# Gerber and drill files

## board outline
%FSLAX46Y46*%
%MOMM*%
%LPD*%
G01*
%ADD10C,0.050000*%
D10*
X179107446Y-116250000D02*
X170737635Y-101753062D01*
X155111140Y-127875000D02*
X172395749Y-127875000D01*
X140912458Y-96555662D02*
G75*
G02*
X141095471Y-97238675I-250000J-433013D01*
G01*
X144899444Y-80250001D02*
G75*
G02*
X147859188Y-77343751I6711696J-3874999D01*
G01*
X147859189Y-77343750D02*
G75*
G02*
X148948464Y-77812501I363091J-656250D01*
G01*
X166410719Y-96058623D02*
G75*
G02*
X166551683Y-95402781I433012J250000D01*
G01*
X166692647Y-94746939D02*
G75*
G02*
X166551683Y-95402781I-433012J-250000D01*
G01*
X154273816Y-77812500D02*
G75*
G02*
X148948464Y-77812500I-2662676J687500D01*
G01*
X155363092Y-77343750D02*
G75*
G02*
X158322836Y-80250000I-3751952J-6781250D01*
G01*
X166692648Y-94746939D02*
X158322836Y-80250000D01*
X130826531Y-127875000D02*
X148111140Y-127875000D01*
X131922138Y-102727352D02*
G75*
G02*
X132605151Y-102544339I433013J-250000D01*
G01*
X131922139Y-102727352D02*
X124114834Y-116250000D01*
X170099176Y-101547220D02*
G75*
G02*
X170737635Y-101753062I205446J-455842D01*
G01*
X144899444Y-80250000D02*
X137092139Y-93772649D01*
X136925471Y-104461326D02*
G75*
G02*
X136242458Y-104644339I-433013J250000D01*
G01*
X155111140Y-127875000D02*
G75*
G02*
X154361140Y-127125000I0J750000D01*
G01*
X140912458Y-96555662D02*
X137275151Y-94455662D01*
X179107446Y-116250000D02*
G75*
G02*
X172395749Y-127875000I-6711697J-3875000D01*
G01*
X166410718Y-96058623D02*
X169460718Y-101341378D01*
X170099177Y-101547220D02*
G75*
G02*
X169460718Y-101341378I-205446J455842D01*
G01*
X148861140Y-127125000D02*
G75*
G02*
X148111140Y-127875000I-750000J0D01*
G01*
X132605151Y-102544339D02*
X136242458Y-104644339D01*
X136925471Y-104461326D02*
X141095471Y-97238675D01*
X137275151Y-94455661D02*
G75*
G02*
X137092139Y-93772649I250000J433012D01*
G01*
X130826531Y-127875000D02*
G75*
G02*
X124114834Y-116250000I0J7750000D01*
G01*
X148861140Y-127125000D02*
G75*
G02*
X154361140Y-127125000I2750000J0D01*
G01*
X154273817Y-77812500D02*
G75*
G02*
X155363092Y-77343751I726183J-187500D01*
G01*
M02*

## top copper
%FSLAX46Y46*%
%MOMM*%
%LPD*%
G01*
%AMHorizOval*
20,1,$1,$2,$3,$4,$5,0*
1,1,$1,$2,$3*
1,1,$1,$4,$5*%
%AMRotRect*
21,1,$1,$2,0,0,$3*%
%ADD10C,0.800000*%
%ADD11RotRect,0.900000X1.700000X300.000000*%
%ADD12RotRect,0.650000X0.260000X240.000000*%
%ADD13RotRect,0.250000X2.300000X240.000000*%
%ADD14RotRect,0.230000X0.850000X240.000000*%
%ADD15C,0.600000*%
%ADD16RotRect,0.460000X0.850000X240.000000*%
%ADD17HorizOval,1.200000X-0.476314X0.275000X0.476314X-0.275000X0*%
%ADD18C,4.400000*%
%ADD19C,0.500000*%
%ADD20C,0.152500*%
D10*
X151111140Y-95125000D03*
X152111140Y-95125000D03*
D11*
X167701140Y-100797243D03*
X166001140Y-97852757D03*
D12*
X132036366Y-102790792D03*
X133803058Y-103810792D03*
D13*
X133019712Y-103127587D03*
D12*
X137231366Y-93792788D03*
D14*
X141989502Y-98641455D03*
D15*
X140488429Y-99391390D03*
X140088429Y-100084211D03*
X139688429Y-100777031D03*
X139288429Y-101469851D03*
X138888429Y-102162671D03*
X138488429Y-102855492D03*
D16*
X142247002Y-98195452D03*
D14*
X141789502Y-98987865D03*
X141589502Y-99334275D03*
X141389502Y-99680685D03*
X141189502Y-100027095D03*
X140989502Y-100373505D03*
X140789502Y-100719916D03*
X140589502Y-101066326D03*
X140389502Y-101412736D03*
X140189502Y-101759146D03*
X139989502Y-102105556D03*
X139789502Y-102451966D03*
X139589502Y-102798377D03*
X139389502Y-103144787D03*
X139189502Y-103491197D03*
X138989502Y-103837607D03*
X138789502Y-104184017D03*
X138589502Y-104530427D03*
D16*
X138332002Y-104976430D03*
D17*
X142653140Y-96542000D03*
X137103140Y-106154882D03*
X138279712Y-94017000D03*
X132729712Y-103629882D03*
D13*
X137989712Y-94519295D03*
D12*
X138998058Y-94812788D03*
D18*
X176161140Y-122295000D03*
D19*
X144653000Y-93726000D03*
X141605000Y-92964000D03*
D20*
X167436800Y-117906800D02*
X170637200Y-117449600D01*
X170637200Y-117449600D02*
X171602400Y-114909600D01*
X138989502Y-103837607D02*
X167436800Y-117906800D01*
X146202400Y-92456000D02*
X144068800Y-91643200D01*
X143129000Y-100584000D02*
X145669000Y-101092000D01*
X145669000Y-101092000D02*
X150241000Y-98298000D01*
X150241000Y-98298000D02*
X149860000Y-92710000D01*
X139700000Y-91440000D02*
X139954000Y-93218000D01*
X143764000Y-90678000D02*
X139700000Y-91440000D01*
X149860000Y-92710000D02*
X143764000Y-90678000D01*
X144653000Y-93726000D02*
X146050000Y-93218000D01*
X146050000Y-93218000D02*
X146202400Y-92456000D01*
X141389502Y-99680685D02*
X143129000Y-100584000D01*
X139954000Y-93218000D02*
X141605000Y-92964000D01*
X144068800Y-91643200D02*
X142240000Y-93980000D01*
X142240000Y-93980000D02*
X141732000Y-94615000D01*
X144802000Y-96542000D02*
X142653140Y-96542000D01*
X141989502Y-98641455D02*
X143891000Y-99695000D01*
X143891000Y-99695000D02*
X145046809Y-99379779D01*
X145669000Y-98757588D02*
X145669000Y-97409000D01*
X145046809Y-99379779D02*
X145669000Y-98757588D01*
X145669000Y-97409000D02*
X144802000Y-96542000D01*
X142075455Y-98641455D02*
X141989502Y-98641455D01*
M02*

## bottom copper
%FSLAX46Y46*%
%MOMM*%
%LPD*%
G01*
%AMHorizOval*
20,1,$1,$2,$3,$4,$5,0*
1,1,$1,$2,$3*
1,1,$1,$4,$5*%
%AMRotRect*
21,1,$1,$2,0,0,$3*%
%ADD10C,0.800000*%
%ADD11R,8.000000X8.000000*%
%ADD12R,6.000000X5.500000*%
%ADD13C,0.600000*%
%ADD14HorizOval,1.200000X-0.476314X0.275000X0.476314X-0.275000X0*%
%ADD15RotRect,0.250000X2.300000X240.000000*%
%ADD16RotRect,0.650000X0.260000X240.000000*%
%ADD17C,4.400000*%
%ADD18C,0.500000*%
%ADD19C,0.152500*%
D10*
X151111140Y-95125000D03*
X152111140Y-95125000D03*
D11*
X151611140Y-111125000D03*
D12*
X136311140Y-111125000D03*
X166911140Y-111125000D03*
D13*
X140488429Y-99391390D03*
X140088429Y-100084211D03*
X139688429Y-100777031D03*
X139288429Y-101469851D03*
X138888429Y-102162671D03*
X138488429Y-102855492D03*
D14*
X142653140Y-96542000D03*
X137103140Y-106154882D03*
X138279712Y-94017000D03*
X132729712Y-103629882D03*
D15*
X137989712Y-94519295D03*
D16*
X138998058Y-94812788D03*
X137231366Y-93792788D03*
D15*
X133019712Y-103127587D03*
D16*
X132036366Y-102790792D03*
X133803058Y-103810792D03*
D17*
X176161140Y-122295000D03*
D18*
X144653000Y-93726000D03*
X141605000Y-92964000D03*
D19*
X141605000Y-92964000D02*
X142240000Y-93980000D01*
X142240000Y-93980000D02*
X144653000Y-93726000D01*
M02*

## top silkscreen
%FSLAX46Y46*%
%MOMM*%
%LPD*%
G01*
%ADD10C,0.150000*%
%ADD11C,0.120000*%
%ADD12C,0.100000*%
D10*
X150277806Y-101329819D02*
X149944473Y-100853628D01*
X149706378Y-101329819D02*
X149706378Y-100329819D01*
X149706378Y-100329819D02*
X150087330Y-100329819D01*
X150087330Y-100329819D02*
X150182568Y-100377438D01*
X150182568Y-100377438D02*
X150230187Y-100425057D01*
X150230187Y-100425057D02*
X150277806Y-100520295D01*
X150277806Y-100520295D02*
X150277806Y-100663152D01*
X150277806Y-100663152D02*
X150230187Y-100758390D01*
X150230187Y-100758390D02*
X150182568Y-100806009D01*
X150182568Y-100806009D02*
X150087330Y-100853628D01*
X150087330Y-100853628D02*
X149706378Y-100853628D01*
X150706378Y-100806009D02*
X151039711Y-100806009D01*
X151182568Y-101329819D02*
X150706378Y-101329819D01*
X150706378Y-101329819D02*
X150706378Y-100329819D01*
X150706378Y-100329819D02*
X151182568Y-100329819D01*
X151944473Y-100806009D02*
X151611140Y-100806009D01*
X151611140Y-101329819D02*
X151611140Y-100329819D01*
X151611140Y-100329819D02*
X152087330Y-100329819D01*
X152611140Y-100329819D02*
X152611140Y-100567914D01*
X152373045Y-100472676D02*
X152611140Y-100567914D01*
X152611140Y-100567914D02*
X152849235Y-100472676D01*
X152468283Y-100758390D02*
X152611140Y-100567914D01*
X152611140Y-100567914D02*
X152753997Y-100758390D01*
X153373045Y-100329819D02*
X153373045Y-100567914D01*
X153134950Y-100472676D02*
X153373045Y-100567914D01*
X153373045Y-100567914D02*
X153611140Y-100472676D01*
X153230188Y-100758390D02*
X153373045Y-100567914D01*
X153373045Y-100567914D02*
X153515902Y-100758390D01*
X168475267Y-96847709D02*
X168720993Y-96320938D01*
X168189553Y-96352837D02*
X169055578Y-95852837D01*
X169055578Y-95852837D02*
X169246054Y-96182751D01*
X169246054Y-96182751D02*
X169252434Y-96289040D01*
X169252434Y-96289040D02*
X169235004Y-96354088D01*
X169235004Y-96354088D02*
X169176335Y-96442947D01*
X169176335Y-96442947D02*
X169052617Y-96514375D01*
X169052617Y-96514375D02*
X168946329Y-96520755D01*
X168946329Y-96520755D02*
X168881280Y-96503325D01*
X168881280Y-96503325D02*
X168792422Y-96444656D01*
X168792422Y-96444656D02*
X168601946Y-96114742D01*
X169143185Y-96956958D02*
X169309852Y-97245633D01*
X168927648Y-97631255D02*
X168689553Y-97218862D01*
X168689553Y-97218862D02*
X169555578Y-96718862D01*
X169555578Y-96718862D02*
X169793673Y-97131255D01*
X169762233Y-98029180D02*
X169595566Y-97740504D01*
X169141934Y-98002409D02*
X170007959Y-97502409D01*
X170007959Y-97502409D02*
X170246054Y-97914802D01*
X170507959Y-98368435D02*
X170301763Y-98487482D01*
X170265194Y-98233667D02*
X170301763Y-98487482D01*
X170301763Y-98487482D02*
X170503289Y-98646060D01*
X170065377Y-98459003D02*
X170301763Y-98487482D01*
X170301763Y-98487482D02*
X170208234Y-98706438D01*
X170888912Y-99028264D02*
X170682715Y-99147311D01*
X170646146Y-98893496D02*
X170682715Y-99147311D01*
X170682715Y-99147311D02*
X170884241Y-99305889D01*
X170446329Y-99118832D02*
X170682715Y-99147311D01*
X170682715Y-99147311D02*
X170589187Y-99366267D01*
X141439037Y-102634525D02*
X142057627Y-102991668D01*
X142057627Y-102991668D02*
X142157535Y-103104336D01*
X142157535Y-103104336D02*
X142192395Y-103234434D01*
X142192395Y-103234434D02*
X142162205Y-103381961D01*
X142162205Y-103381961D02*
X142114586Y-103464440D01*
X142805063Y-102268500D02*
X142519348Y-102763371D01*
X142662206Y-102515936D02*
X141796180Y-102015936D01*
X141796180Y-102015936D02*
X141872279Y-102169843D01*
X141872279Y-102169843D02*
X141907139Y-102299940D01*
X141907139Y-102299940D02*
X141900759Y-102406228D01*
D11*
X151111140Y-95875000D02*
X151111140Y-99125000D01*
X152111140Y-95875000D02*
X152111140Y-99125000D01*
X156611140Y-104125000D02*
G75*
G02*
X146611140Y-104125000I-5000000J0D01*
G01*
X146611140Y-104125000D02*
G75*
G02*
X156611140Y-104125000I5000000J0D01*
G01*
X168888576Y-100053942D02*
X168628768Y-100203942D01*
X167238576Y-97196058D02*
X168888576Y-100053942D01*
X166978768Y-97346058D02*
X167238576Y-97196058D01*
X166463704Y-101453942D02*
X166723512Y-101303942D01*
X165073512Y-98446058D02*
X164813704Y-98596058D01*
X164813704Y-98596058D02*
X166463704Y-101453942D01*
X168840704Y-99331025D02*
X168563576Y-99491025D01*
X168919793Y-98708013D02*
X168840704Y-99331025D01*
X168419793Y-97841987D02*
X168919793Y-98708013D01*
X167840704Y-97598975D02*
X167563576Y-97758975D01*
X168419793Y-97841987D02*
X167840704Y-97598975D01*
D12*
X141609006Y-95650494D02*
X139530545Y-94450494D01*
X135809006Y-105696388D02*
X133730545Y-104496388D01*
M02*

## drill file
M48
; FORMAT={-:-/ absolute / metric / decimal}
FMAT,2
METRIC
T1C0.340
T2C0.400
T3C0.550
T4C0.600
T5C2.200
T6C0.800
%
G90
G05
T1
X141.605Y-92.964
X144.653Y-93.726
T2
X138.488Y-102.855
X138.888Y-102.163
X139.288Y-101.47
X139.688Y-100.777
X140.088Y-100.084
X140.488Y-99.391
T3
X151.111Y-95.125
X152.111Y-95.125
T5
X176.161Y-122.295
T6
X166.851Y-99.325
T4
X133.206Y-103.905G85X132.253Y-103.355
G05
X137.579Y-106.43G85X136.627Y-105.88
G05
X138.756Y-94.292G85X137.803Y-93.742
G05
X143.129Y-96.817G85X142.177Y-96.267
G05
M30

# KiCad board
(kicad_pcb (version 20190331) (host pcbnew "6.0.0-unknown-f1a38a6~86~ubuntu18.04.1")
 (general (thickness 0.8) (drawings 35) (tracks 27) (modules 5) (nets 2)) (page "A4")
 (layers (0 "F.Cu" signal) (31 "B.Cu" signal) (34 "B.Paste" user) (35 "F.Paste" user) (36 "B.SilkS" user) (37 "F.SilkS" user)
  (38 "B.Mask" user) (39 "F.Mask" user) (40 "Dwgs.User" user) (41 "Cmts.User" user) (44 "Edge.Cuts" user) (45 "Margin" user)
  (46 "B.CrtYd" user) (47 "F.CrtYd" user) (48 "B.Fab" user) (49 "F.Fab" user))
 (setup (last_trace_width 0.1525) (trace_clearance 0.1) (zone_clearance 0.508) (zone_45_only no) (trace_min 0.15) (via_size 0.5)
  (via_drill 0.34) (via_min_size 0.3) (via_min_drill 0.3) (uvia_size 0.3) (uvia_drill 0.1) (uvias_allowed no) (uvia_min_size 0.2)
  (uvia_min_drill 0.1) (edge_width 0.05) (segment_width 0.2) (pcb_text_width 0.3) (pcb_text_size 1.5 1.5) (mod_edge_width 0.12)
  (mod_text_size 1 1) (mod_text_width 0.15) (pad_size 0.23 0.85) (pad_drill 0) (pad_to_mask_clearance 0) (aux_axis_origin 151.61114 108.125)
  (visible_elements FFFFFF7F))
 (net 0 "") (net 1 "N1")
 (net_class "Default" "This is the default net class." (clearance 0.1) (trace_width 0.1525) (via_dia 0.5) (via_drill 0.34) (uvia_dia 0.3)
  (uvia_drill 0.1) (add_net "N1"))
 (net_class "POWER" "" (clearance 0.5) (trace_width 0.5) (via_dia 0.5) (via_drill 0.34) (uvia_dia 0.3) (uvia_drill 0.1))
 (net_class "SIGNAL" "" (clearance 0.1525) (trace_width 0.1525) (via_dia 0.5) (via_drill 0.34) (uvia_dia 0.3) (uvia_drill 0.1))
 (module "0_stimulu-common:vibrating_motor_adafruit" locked (layer "F.Cu") (at 151.61114 104.125 180)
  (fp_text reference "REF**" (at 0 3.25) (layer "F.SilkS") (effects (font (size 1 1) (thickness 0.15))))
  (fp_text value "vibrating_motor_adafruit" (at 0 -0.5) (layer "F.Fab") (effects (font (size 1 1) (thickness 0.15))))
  (fp_line (start 0.5 8.25) (end 0.5 5) (layer "F.SilkS") (width 0.12))
  (fp_line (start -0.5 8.25) (end -0.5 5) (layer "F.SilkS") (width 0.12))
  (fp_circle (center 0 0) (end 3 -4) (layer "F.SilkS") (width 0.12))
  (pad "2" thru_hole circle (at 0.5 9 180) (size 0.8 0.8) (drill 0.55) (layers *.Cu *.Mask))
  (pad "1" thru_hole circle (at -0.5 9 180) (size 0.8 0.8) (drill 0.55) (layers *.Cu *.Mask)))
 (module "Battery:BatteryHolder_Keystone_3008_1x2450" (layer "B.Cu") (at 151.61114 111.125 180)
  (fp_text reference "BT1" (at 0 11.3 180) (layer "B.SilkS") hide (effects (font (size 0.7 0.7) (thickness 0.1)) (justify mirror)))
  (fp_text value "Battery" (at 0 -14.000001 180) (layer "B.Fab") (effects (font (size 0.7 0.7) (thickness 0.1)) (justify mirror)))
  (pad "2" smd rect (at 0 0 180) (size 8 8) (layers "B.Cu" "B.Mask"))
  (pad "1" smd rect (at 15.3 0 180) (size 6 5.5) (layers "B.Cu" "B.Paste" "B.Mask"))
  (pad "1" smd rect (at -15.3 0 180) (size 6 5.5) (layers "B.Cu" "B.Paste" "B.Mask")))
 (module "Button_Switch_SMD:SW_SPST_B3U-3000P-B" (layer "F.Cu") (at 166.85114 99.325 300)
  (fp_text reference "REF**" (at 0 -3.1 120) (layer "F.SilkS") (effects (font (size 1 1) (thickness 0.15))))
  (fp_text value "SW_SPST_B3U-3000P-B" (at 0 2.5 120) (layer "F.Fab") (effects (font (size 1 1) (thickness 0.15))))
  (fp_line (start 1.65 -1.4) (end 1.65 -1.1) (layer "F.SilkS") (width 0.12))
  (fp_line (start -1.65 -1.4) (end 1.65 -1.4) (layer "F.SilkS") (width 0.12))
  (fp_line (start -1.65 -1.1) (end -1.65 -1.4) (layer "F.SilkS") (width 0.12))
  (fp_line (start 1.65 1.4) (end 1.65 1.1) (layer "F.SilkS") (width 0.12))
  (fp_line (start -1.65 1.1) (end -1.65 1.4) (layer "F.SilkS") (width 0.12))
  (fp_line (start -1.65 1.4) (end 1.65 1.4) (layer "F.SilkS") (width 0.12))
  (fp_line (start 1 -1.72) (end 1 -1.4) (layer "F.SilkS") (width 0.12))
  (fp_line (start 0.5 -2.1) (end 1 -1.72) (layer "F.SilkS") (width 0.12))
  (fp_line (start -0.5 -2.1) (end 0.5 -2.1) (layer "F.SilkS") (width 0.12))
  (fp_line (start -1 -1.72) (end -1 -1.4) (layer "F.SilkS") (width 0.12))
  (fp_line (start -0.5 -2.1) (end -1 -1.72) (layer "F.SilkS") (width 0.12))
  (pad "" np_thru_hole circle (at 0 0 300) (size 0.8 0.8) (drill 0.8) (layers *.Cu *.Mask))
  (pad "2" smd rect (at 1.7 0 300) (size 0.9 1.7) (layers "F.Cu" "F.Paste" "F.Mask"))
  (pad "1" smd rect (at -1.7 0 300) (size 0.9 1.7) (layers "F.Cu" "F.Paste" "F.Mask") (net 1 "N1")))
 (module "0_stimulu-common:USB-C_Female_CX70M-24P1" (layer "F.Cu") (at 139.488429 101.123441 240)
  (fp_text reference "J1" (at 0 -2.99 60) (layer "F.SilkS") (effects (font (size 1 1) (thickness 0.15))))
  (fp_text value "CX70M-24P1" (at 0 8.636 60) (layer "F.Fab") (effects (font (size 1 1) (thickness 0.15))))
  (fp_line (start -5.8 0.9) (end -5.8 3.3) (layer "F.SilkS") (width 0.1))
  (fp_line (start 5.8 0.9) (end 5.8 3.3) (layer "F.SilkS") (width 0.1))
  (pad "SH" smd rect (at 5.17 5.62 240) (size 0.65 0.26) (layers "F.Cu" "F.Paste" "F.Mask") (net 1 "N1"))
  (pad "SH" smd rect (at 5.17 3.58 240) (size 0.65 0.26) (layers "F.Cu" "F.Paste" "F.Mask") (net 1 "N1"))
  (pad "SH" smd rect (at 4.97 4.6 240) (size 0.25 2.3) (layers "F.Cu" "F.Paste" "F.Mask") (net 1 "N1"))
  (pad "SH" smd rect (at -5.22 5.62 240) (size 0.65 0.26) (layers "F.Cu" "F.Paste" "F.Mask") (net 1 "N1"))
  (pad "B12" smd rect (at -3.399999 -0.925 240) (size 0.23 0.85) (layers "F.Cu" "F.Paste" "F.Mask") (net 1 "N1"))
  (pad "B9" thru_hole circle (at -2 0 240) (size 0.6 0.6) (drill 0.4) (layers *.Cu *.Mask))
  (pad "B8" thru_hole circle (at -1.2 0 240) (size 0.6 0.6) (drill 0.4) (layers *.Cu *.Mask))
  (pad "B7" thru_hole circle (at -0.4 0 240) (size 0.6 0.6) (drill 0.4) (layers *.Cu *.Mask))
  (pad "B6" thru_hole circle (at 0.4 0 240) (size 0.6 0.6) (drill 0.4) (layers *.Cu *.Mask))
  (pad "B5" thru_hole circle (at 1.2 0 240) (size 0.6 0.6) (drill 0.4) (layers *.Cu *.Mask))
  (pad "B4" thru_hole circle (at 2 0 240) (size 0.6 0.6) (drill 0.4) (layers *.Cu *.Mask))
  (pad "" smd rect (at -3.915 -0.925 240) (size 0.46 0.85) (layers "F.Cu" "F.Paste" "F.Mask"))
  (pad "B11" smd rect (at -3 -0.925 240) (size 0.23 0.85) (layers "F.Cu" "F.Paste" "F.Mask"))
  (pad "B10" smd rect (at -2.6 -0.925 240) (size 0.23 0.85) (layers "F.Cu" "F.Paste" "F.Mask"))
  (pad "A1" smd rect (at -2.2 -0.925 240) (size 0.23 0.85) (layers "F.Cu" "F.Paste" "F.Mask"))
  (pad "A2" smd rect (at -1.8 -0.925 240) (size 0.23 0.85) (layers "F.Cu" "F.Paste" "F.Mask"))
  (pad "A3" smd rect (at -1.4 -0.925 240) (size 0.23 0.85) (layers "F.Cu" "F.Paste" "F.Mask"))
  (pad "A4" smd rect (at -1 -0.925 240) (size 0.23 0.85) (layers "F.Cu" "F.Paste" "F.Mask"))
  (pad "A5" smd rect (at -0.6 -0.925 240) (size 0.23 0.85) (layers "F.Cu" "F.Paste" "F.Mask"))
  (pad "A6" smd rect (at -0.2 -0.925 240) (size 0.23 0.85) (layers "F.Cu" "F.Paste" "F.Mask"))
  (pad "A7" smd rect (at 0.2 -0.925 240) (size 0.23 0.85) (layers "F.Cu" "F.Paste" "F.Mask"))
  (pad "A8" smd rect (at 0.6 -0.925 240) (size 0.23 0.85) (layers "F.Cu" "F.Paste" "F.Mask"))
  (pad "A9" smd rect (at 1 -0.925 240) (size 0.23 0.85) (layers "F.Cu" "F.Paste" "F.Mask"))
  (pad "A10" smd rect (at 1.4 -0.925 240) (size 0.23 0.85) (layers "F.Cu" "F.Paste" "F.Mask"))
  (pad "A11" smd rect (at 1.8 -0.925 240) (size 0.23 0.85) (layers "F.Cu" "F.Paste" "F.Mask"))
  (pad "A12" smd rect (at 2.2 -0.925 240) (size 0.23 0.85) (layers "F.Cu" "F.Paste" "F.Mask"))
  (pad "B3" smd rect (at 2.6 -0.925 240) (size 0.23 0.85) (layers "F.Cu" "F.Paste" "F.Mask"))
  (pad "B2" smd rect (at 3 -0.925 240) (size 0.23 0.85) (layers "F.Cu" "F.Paste" "F.Mask"))
  (pad "B1" smd rect (at 3.4 -0.925 240) (size 0.23 0.85) (layers "F.Cu" "F.Paste" "F.Mask"))
  (pad "" smd rect (at 3.915 -0.925 240) (size 0.46 0.85) (layers "F.Cu" "F.Paste" "F.Mask"))
  (pad "SH" thru_hole oval (at -5.55 -0.45 240) (size 1.2 2.3) (drill oval 0.6 1.7) (layers *.Cu *.Mask) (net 1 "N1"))
  (pad "SH" thru_hole oval (at 5.55 -0.45 240) (size 1.2 2.3) (drill oval 0.6 1.7) (layers *.Cu *.Mask) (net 1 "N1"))
  (pad "SH" thru_hole oval (at -5.55 4.6 240) (size 1.2 2.3) (drill oval 0.6 1.7) (layers *.Cu *.Mask) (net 1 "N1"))
  (pad "SH" thru_hole oval (at 5.55 4.6 240) (size 1.2 2.3) (drill oval 0.6 1.7) (layers *.Cu *.Mask) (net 1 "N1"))
  (pad "SH" smd rect (at -4.97 4.6 240) (size 0.25 2.3) (layers "F.Cu" "F.Paste" "F.Mask") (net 1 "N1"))
  (pad "SH" smd rect (at -5.22 3.58 240) (size 0.65 0.26) (layers "F.Cu" "F.Paste" "F.Mask") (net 1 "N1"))
  (pad "SH" smd rect (at -4.97 4.6 240) (size 0.25 2.3) (layers "B.Cu" "B.Paste" "B.Mask") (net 1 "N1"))
  (pad "SH" smd rect (at -5.22 3.58 240) (size 0.65 0.26) (layers "B.Cu" "B.Paste" "B.Mask") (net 1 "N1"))
  (pad "SH" smd rect (at -5.22 5.62 240) (size 0.65 0.26) (layers "B.Cu" "B.Paste" "B.Mask") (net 1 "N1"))
  (pad "SH" smd rect (at 4.97 4.6 240) (size 0.25 2.3) (layers "B.Cu" "B.Paste" "B.Mask") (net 1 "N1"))
  (pad "SH" smd rect (at 5.17 5.62 240) (size 0.65 0.26) (layers "B.Cu" "B.Paste" "B.Mask") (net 1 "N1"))
  (pad "SH" smd rect (at 5.17 3.58 240) (size 0.65 0.26) (layers "B.Cu" "B.Paste" "B.Mask") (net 1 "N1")))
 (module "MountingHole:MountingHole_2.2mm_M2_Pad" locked (layer "F.Cu") (at 176.16114 122.295)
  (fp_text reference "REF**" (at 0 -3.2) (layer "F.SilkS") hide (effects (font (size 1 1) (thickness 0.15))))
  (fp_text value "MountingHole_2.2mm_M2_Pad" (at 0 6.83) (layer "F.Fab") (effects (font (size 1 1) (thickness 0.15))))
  (pad "1" thru_hole circle (at 0 0) (size 4.4 4.4) (drill 2.2) (layers *.Cu *.Mask)))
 (gr_line (start 179.107446 116.25) (end 170.737635 101.753062) (layer "Edge.Cuts") (width 0.05))
 (gr_line (start 155.11114 127.875) (end 172.395749 127.875) (layer "Edge.Cuts") (width 0.05))
 (gr_arc (start 140.662458 96.988675) (end 141.095471 97.238675) (angle -90) (layer "Edge.Cuts") (width 0.05))
 (gr_arc (start 151.61114 84.125) (end 147.859188 77.343751) (angle -31.04497563) (layer "Edge.Cuts") (width 0.05))
 (gr_arc (start 148.22228 78) (end 148.948464 77.812501) (angle -104.4775122) (layer "Edge.Cuts") (width 0.05))
 (gr_arc (start 166.843731 95.808623) (end 166.551683 95.402781) (angle -84.26082952) (layer "Edge.Cuts") (width 0.05))
 (gr_arc (start 166.259635 94.996939) (end 166.551683 95.402781) (angle -84.26082952) (layer "Edge.Cuts") (width 0.05))
 (gr_arc (start 151.61114 77.125) (end 148.948464 77.8125) (angle -151.0449756) (layer "Edge.Cuts") (width 0.05))
 (gr_arc (start 151.61114 84.125) (end 158.322836 80.25) (angle -31.04497563) (layer "Edge.Cuts") (width 0.05))
 (gr_line (start 166.692648 94.746939) (end 158.322836 80.25) (layer "Edge.Cuts") (width 0.05))
 (gr_line (start 130.826531 127.875) (end 148.11114 127.875) (layer "Edge.Cuts") (width 0.05))
 (gr_arc (start 132.355151 102.977352) (end 132.605151 102.544339) (angle -90) (layer "Edge.Cuts") (width 0.05))
 (gr_line (start 131.922139 102.727352) (end 124.114834 116.25) (layer "Edge.Cuts") (width 0.05))
 (gr_arc (start 170.304622 102.003062) (end 170.737635 101.753062) (angle -84.26082952) (layer "Edge.Cuts") (width 0.05))
 (gr_line (start 144.899444 80.25) (end 137.092139 93.772649) (layer "Edge.Cuts") (width 0.05))
 (gr_arc (start 136.492458 104.211326) (end 136.242458 104.644339) (angle -90) (layer "Edge.Cuts") (width 0.05))
 (gr_arc (start 155.11114 127.125) (end 154.36114 127.125) (angle -90) (layer "Edge.Cuts") (width 0.05))
 (gr_line (start 140.912458 96.555662) (end 137.275151 94.455662) (layer "Edge.Cuts") (width 0.05))
 (gr_arc (start 172.395749 120.125) (end 172.395749 127.875) (angle -120) (layer "Edge.Cuts") (width 0.05))
 (gr_line (start 166.410718 96.058623) (end 169.460718 101.341378) (layer "Edge.Cuts") (width 0.05))
 (gr_arc (start 169.893731 101.091378) (end 169.460718 101.341378) (angle -84.26082952) (layer "Edge.Cuts") (width 0.05))
 (gr_arc (start 148.11114 127.125) (end 148.11114 127.875) (angle -90) (layer "Edge.Cuts") (width 0.05))
 (gr_line (start 132.605151 102.544339) (end 136.242458 104.644339) (layer "Edge.Cuts") (width 0.05))
 (gr_line (start 136.925471 104.461326) (end 141.095471 97.238675) (layer "Edge.Cuts") (width 0.05))
 (gr_arc (start 137.525151 94.022649) (end 137.092139 93.772649) (angle -90) (layer "Edge.Cuts") (width 0.05))
 (gr_arc (start 130.826531 120.125) (end 124.114834 116.25) (angle -120) (layer "Edge.Cuts") (width 0.05))
 (gr_arc (start 151.61114 127.125) (end 154.36114 127.125) (angle -180) (layer "Edge.Cuts") (width 0.05))
 (gr_arc (start 155 78) (end 155.363092 77.343751) (angle -104.4775122) (layer "Edge.Cuts") (width 0.05))
 (segment (start 167.4368 117.9068) (end 170.6372 117.4496) (width 0.1525) (layer "F.Cu") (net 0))
 (segment (start 170.6372 117.4496) (end 171.6024 114.9096) (width 0.1525) (layer "F.Cu") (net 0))
 (segment (start 138.989502 103.837607) (end 167.4368 117.9068) (width 0.1525) (layer "F.Cu") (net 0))
 (segment (start 146.2024 92.456) (end 144.0688 91.6432) (width 0.1525) (layer "F.Cu") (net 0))
 (via (at 144.653 93.726) (size 0.5) (drill 0.34) (layers "F.Cu" "B.Cu") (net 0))
 (segment (start 143.129 100.584) (end 145.669 101.092) (width 0.1525) (layer "F.Cu") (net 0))
 (segment (start 145.669 101.092) (end 150.241 98.298) (width 0.1525) (layer "F.Cu") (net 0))
 (segment (start 150.241 98.298) (end 149.86 92.71) (width 0.1525) (layer "F.Cu") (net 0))
 (segment (start 139.7 91.44) (end 139.954 93.218) (width 0.1525) (layer "F.Cu") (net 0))
 (segment (start 143.764 90.678) (end 139.7 91.44) (width 0.1525) (layer "F.Cu") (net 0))
 (via (at 141.605 92.964) (size 0.5) (drill 0.34) (layers "F.Cu" "B.Cu") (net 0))
 (segment (start 149.86 92.71) (end 143.764 90.678) (width 0.1525) (layer "F.Cu") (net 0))
 (segment (start 144.653 93.726) (end 146.05 93.218) (width 0.1525) (layer "F.Cu") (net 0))
 (segment (start 146.05 93.218) (end 146.2024 92.456) (width 0.1525) (layer "F.Cu") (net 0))
 (segment (start 141.389502 99.680685) (end 143.129 100.584) (width 0.1525) (layer "F.Cu") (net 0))
 (segment (start 139.954 93.218) (end 141.605 92.964) (width 0.1525) (layer "F.Cu") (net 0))
 (segment (start 141.605 92.964) (end 142.24 93.98) (width 0.1525) (layer "B.Cu") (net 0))
 (segment (start 142.24 93.98) (end 144.653 93.726) (width 0.1525) (layer "B.Cu") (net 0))
 (segment (start 144.0688 91.6432) (end 142.24 93.98) (width 0.1525) (layer "F.Cu") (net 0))
 (segment (start 142.24 93.98) (end 141.732 94.615) (width 0.1525) (layer "F.Cu") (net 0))
 (segment (start 144.802 96.542) (end 142.65314 96.542) (width 0.1525) (layer "F.Cu") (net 1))
 (segment (start 141.989502 98.641455) (end 143.891 99.695) (width 0.1525) (layer "F.Cu") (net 1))
 (segment (start 143.891 99.695) (end 145.046809 99.379779) (width 0.1525) (layer "F.Cu") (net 1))
 (segment (start 145.669 98.757588) (end 145.669 97.409) (width 0.1525) (layer "F.Cu") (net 1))
 (segment (start 145.046809 99.379779) (end 145.669 98.757588) (width 0.1525) (layer "F.Cu") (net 1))
 (segment (start 145.669 97.409) (end 144.802 96.542) (width 0.1525) (layer "F.Cu") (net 1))
 (segment (start 142.075455 98.641455) (end 141.989502 98.641455) (width 0.1525) (layer "F.Cu") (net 1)))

